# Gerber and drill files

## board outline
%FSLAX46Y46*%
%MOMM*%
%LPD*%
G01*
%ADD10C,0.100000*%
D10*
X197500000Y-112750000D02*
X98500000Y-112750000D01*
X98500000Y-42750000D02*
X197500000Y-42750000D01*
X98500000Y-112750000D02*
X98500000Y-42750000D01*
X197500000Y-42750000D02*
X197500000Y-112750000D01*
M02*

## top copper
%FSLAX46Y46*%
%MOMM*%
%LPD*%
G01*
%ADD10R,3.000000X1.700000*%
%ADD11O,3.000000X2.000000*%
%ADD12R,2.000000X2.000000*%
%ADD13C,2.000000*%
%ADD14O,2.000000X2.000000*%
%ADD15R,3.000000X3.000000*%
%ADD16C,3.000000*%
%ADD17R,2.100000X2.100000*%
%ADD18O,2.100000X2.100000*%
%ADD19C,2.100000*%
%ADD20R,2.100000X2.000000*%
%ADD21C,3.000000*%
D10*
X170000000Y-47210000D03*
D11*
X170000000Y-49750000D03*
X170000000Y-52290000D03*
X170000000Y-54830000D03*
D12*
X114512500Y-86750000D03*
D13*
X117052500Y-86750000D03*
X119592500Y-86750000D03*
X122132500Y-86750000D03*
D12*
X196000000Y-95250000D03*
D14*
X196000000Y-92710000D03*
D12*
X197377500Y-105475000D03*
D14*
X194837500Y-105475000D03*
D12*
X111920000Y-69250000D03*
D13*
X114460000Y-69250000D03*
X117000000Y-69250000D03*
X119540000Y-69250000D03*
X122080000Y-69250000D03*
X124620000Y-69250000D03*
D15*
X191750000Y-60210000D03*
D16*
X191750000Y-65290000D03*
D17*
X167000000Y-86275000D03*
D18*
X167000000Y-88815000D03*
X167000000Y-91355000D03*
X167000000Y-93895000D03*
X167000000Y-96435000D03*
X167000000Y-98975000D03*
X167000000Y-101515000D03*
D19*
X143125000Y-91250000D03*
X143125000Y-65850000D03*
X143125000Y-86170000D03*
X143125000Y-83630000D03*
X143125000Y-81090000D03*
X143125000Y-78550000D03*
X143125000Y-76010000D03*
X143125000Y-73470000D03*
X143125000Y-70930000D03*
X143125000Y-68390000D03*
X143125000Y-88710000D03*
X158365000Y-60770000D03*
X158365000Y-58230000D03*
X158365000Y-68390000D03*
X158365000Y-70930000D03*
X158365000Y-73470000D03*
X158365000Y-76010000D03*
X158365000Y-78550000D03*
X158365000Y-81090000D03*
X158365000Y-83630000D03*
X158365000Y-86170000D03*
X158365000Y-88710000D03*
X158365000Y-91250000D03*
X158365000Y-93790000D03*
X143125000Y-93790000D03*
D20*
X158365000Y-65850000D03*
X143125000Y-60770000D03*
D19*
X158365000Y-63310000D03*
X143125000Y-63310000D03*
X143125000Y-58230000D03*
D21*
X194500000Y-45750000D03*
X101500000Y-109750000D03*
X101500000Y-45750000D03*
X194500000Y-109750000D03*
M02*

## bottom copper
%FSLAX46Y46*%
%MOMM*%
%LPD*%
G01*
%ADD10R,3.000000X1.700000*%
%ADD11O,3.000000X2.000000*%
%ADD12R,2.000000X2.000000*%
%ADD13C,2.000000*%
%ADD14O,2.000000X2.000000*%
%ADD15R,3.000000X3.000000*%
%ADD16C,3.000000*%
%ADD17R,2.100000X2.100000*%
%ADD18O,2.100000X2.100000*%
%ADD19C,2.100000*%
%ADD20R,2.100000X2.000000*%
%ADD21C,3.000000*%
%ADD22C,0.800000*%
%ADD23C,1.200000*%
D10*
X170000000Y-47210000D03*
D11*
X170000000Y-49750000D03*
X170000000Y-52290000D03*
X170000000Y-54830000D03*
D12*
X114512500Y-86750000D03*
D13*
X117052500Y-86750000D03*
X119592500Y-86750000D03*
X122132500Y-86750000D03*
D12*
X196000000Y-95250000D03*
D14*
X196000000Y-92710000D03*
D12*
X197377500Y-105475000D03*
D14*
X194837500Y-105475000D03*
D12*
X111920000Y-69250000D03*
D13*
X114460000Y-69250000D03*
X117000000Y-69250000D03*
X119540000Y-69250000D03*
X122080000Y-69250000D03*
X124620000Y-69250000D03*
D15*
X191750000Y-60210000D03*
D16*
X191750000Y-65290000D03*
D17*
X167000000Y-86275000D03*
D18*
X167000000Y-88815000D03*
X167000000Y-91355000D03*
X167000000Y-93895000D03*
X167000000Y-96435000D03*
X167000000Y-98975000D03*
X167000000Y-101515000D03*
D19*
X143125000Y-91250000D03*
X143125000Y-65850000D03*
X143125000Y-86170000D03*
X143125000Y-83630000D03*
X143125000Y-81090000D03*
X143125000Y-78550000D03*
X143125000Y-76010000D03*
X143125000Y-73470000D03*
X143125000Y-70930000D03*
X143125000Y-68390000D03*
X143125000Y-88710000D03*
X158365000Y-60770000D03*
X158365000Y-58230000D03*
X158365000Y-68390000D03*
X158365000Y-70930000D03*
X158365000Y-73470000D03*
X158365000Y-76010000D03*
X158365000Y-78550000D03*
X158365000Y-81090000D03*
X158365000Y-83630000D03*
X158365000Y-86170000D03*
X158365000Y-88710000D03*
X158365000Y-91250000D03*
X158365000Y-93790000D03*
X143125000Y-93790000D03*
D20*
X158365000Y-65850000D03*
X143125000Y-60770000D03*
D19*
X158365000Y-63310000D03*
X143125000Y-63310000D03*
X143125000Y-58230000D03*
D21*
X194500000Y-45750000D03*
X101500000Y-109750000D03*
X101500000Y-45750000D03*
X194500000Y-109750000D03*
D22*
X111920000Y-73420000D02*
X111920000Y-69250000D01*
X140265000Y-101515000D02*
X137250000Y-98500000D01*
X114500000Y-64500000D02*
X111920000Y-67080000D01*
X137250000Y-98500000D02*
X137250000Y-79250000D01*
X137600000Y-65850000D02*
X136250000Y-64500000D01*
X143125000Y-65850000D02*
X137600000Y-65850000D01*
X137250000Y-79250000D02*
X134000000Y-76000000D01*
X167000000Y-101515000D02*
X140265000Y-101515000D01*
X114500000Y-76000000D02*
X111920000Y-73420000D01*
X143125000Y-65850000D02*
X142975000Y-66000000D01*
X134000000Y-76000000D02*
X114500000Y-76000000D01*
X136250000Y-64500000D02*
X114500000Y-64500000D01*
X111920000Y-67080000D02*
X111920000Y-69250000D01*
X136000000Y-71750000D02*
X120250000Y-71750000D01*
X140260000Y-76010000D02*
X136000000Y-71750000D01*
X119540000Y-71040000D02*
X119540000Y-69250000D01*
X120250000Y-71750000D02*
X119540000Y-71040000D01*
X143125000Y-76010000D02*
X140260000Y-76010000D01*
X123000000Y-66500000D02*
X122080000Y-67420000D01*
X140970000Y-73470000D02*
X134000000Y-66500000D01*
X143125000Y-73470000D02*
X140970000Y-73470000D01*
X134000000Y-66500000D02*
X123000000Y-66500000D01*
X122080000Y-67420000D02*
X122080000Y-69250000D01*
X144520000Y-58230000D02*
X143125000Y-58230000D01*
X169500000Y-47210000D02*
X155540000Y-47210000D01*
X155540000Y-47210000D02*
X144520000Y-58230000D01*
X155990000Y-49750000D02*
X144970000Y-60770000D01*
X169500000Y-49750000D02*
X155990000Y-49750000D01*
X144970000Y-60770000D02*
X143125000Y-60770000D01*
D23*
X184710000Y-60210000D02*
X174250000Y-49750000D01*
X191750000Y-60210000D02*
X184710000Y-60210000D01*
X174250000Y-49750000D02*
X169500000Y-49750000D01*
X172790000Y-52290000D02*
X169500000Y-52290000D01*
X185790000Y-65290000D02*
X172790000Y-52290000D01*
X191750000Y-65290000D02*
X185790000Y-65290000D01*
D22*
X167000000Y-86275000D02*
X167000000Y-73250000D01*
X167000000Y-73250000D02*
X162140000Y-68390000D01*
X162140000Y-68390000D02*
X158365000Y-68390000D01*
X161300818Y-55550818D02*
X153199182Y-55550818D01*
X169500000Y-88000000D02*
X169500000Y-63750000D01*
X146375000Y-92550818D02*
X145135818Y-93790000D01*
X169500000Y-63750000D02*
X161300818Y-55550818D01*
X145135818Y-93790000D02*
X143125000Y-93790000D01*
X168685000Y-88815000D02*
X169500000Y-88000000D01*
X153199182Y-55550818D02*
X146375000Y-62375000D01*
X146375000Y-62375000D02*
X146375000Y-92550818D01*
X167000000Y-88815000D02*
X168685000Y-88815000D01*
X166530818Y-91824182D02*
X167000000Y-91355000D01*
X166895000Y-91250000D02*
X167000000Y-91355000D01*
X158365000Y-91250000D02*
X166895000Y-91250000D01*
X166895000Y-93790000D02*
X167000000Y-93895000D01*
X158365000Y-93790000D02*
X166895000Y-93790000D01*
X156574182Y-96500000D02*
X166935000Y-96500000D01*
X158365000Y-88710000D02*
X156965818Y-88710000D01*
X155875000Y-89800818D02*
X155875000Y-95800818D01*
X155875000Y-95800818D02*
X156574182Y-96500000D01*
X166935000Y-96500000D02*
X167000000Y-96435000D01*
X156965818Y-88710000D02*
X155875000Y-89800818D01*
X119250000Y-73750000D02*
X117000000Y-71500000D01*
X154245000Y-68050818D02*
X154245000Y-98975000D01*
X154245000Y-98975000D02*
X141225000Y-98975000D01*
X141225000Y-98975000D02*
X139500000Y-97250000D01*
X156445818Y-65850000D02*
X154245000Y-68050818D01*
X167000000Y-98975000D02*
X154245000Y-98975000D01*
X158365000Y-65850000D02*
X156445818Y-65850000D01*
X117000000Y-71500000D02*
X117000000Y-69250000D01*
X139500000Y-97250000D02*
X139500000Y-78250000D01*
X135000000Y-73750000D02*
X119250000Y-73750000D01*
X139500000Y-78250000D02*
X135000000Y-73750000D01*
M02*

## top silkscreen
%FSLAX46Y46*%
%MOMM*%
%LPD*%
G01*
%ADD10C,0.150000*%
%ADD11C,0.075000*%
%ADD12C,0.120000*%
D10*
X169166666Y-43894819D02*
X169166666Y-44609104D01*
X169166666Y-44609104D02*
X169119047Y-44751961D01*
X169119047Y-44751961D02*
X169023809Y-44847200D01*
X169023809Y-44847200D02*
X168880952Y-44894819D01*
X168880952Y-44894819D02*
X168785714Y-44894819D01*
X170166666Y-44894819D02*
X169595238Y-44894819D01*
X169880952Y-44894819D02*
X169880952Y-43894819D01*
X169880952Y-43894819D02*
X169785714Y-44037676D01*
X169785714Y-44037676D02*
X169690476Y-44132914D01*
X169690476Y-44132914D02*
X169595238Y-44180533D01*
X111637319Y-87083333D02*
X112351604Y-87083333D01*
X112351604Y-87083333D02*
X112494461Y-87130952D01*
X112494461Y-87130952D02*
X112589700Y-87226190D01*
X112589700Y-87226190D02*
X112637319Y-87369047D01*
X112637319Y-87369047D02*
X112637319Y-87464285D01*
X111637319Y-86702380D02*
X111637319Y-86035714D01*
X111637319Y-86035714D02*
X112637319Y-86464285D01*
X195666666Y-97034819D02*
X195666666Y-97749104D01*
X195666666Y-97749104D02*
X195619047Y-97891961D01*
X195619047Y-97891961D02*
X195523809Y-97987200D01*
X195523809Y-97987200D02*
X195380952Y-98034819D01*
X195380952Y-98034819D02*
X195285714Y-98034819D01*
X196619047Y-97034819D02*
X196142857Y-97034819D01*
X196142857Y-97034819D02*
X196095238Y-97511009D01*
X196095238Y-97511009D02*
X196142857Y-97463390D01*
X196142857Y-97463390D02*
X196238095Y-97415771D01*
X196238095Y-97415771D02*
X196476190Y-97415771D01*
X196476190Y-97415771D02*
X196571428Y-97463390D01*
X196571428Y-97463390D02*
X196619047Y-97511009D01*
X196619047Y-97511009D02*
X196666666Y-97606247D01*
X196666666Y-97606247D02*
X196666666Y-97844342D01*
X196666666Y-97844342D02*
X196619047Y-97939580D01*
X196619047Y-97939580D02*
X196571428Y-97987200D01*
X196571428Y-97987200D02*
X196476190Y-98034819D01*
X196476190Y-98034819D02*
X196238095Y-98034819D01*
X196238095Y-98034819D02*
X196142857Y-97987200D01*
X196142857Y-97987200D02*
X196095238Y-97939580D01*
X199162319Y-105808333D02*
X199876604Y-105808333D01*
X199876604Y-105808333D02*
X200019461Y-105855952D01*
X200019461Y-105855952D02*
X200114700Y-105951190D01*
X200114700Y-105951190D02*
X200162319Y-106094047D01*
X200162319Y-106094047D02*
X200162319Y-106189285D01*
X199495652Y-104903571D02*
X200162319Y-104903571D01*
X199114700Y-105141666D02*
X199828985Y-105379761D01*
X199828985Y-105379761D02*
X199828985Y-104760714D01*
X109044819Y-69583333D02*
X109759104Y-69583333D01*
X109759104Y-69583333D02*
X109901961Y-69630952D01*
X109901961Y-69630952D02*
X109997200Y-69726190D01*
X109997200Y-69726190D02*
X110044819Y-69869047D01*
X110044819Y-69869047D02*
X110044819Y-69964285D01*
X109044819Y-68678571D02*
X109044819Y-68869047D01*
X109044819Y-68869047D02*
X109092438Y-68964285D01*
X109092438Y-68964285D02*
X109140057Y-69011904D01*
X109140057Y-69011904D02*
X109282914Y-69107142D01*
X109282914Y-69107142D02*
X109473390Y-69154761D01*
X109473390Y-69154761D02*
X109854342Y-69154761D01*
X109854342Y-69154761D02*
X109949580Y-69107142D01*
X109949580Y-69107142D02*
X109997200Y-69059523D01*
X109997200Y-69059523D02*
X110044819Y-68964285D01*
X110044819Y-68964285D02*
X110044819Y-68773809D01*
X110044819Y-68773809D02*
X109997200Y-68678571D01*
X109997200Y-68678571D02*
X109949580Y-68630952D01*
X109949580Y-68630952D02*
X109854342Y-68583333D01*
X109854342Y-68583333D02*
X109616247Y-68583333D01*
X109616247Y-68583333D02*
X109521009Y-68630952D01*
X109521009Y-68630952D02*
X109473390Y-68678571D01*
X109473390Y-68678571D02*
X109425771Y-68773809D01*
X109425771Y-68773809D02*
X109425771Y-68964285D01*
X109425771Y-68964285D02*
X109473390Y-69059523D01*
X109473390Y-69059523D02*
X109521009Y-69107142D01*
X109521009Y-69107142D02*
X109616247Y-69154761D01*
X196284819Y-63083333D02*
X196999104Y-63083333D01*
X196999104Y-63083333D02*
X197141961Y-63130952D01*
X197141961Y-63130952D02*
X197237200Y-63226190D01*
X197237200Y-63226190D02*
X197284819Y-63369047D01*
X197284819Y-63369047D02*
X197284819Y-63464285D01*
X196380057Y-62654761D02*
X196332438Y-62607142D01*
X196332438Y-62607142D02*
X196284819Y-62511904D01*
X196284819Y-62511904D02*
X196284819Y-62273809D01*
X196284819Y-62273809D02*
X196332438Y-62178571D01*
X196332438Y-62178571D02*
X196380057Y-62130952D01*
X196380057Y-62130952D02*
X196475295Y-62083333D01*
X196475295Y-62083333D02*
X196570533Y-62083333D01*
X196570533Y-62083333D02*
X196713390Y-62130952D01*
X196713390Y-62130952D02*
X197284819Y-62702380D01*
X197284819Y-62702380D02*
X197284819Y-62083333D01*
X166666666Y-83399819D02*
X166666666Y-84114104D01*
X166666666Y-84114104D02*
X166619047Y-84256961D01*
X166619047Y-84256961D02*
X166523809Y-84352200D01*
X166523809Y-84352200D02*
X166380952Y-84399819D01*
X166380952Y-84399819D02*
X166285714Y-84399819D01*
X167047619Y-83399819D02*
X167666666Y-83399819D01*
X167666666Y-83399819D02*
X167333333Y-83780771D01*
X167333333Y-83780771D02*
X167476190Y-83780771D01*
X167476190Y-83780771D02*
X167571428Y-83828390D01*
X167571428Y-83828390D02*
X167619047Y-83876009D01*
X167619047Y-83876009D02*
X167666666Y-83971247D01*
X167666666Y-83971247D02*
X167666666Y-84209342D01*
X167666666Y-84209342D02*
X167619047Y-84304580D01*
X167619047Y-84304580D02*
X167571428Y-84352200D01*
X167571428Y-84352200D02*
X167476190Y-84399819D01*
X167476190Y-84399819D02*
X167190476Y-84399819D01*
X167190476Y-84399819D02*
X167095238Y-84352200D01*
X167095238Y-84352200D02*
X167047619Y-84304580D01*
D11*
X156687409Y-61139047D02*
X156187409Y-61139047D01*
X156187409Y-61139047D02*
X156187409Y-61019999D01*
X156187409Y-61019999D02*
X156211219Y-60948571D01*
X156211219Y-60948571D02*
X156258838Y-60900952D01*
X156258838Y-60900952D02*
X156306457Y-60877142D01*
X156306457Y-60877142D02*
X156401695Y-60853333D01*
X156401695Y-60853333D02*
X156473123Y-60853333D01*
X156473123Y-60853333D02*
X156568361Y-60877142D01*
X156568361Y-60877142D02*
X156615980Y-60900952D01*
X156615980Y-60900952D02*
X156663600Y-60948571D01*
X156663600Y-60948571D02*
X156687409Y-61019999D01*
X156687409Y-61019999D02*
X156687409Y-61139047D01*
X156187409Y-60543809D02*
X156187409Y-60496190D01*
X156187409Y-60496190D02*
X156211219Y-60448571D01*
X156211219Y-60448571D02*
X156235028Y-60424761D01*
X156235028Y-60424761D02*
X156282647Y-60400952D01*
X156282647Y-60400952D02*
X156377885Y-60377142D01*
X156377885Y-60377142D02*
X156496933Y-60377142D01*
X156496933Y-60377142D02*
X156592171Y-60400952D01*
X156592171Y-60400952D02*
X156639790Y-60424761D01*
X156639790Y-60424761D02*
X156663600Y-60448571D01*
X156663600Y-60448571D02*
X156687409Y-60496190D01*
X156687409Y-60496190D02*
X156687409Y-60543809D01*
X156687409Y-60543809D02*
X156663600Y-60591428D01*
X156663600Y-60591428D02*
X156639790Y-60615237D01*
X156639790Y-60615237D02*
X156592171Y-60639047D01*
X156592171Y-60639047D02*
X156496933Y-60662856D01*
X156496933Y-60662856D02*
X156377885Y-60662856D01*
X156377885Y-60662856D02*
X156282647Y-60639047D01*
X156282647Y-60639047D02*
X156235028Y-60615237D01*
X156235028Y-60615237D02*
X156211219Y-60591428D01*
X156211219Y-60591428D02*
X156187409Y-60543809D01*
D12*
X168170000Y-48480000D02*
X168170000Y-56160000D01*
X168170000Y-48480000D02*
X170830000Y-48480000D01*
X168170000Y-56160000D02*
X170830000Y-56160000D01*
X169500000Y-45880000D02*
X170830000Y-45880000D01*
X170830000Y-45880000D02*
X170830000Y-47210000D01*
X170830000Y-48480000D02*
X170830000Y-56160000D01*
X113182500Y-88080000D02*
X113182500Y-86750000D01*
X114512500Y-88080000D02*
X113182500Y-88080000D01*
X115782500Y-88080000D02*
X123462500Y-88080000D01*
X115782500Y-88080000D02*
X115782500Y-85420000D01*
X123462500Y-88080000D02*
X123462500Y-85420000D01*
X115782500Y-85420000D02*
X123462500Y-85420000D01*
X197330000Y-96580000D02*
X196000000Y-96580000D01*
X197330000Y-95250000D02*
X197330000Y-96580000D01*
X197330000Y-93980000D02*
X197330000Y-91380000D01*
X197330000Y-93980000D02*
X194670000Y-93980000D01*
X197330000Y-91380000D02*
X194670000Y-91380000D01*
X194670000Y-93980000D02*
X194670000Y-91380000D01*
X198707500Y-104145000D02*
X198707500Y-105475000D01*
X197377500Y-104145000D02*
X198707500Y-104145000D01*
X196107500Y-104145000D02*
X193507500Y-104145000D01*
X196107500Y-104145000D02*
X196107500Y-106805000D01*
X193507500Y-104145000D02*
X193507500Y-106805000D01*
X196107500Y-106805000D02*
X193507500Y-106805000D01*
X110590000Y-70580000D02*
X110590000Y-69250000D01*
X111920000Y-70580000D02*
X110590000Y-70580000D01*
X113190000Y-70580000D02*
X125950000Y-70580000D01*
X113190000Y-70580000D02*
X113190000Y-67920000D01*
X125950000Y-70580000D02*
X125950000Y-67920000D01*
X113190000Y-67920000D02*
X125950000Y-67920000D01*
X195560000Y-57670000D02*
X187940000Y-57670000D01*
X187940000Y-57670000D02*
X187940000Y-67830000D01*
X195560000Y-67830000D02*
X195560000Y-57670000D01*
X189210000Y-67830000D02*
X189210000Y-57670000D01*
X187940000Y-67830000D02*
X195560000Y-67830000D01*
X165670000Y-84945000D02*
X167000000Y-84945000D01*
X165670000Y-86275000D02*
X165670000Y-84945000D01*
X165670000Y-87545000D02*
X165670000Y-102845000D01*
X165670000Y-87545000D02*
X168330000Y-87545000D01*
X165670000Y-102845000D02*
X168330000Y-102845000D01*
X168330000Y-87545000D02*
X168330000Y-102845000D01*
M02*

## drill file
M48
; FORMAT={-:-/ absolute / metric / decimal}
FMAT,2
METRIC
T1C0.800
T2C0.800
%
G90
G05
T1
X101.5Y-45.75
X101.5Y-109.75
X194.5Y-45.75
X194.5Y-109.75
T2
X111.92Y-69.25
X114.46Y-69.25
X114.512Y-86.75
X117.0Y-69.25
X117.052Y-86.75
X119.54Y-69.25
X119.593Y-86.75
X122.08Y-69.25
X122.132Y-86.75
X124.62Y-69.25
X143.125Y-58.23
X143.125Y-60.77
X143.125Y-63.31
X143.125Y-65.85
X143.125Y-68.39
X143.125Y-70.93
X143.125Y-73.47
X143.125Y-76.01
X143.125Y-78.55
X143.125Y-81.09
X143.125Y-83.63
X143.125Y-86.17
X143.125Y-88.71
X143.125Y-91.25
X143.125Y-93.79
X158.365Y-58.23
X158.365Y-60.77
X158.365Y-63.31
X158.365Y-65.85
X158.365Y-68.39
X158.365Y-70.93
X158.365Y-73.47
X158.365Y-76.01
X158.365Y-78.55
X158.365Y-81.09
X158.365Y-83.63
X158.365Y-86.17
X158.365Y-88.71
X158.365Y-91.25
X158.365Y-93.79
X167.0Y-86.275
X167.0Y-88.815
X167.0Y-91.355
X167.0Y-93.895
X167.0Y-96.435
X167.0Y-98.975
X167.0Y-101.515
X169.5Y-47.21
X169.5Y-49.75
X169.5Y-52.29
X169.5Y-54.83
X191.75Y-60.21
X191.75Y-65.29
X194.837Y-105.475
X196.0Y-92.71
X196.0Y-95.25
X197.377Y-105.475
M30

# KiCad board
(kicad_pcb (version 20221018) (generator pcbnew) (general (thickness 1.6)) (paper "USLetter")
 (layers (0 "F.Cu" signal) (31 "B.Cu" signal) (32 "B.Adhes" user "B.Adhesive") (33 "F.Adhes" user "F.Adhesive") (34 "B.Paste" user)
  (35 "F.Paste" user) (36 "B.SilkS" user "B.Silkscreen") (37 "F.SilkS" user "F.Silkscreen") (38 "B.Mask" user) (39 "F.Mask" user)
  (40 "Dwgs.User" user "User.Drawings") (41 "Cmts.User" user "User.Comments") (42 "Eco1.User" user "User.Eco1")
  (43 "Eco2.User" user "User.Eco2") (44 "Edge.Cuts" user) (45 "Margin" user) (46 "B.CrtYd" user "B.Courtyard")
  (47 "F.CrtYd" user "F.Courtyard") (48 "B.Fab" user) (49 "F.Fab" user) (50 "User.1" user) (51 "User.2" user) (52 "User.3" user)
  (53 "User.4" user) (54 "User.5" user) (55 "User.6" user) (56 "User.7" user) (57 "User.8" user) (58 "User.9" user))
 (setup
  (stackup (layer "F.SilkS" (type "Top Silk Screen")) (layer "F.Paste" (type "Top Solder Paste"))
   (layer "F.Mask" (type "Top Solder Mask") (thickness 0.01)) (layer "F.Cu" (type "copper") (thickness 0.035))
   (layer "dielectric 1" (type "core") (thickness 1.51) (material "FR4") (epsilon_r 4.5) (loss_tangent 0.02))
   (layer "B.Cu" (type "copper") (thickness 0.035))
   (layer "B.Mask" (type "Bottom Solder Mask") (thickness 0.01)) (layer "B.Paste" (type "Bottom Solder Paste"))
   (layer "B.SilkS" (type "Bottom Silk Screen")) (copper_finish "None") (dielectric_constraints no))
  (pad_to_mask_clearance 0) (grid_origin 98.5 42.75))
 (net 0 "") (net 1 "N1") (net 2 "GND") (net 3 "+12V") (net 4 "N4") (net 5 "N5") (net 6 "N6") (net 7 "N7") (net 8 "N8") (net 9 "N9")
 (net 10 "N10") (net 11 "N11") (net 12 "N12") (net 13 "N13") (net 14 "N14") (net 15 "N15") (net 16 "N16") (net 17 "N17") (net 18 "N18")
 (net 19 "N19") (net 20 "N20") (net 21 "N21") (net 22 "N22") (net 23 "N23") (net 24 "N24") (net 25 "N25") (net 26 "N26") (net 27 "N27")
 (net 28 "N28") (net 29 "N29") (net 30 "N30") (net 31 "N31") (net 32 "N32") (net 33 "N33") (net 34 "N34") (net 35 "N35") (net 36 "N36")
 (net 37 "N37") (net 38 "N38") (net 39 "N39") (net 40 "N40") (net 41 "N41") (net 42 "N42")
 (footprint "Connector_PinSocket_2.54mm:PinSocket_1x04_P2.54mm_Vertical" (layer "F.Cu") (at 169.5 47.21)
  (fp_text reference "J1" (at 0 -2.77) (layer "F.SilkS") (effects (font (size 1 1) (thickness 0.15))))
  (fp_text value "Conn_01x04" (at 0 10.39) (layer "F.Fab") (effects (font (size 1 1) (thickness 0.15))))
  (fp_line (start -1.33 1.27) (end -1.33 8.95) (stroke (width 0.12) (type solid)) (layer "F.SilkS"))
  (fp_line (start -1.33 1.27) (end 1.33 1.27) (stroke (width 0.12) (type solid)) (layer "F.SilkS"))
  (fp_line (start -1.33 8.95) (end 1.33 8.95) (stroke (width 0.12) (type solid)) (layer "F.SilkS"))
  (fp_line (start 0 -1.33) (end 1.33 -1.33) (stroke (width 0.12) (type solid)) (layer "F.SilkS"))
  (fp_line (start 1.33 -1.33) (end 1.33 0) (stroke (width 0.12) (type solid)) (layer "F.SilkS"))
  (fp_line (start 1.33 1.27) (end 1.33 8.95) (stroke (width 0.12) (type solid)) (layer "F.SilkS"))
  (pad "1" thru_hole rect (at 0 0) (size 3 1.7) (drill 0.8 (offset 0.5 0)) (layers "*.Cu" "*.Mask") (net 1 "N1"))
  (pad "2" thru_hole oval (at 0 2.54) (size 3 2) (drill 0.8 (offset 0.5 0)) (layers "*.Cu" "*.Mask") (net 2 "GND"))
  (pad "3" thru_hole oval (at 0 5.08) (size 3 2) (drill 0.8 (offset 0.5 0)) (layers "*.Cu" "*.Mask") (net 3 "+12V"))
  (pad "4" thru_hole oval (at 0 7.62) (size 3 2) (drill 0.8 (offset 0.5 0)) (layers "*.Cu" "*.Mask") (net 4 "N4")))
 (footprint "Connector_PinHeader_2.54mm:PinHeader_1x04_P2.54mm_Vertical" (layer "F.Cu") (at 114.5125 86.75 90)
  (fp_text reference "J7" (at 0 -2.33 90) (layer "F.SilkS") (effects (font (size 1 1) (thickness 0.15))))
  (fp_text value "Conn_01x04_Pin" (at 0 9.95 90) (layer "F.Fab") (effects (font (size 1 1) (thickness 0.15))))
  (fp_line (start -1.33 -1.33) (end 0 -1.33) (stroke (width 0.12) (type solid)) (layer "F.SilkS"))
  (fp_line (start -1.33 0) (end -1.33 -1.33) (stroke (width 0.12) (type solid)) (layer "F.SilkS"))
  (fp_line (start -1.33 1.27) (end -1.33 8.95) (stroke (width 0.12) (type solid)) (layer "F.SilkS"))
  (fp_line (start -1.33 1.27) (end 1.33 1.27) (stroke (width 0.12) (type solid)) (layer "F.SilkS"))
  (fp_line (start -1.33 8.95) (end 1.33 8.95) (stroke (width 0.12) (type solid)) (layer "F.SilkS"))
  (fp_line (start 1.33 1.27) (end 1.33 8.95) (stroke (width 0.12) (type solid)) (layer "F.SilkS"))
  (pad "1" thru_hole rect (at 0 0 90) (size 2 2) (drill 0.8) (layers "*.Cu" "*.Mask") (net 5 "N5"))
  (pad "2" thru_hole circle (at 0 2.54 90) (size 2 2) (drill 0.8) (layers "*.Cu" "*.Mask") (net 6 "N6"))
  (pad "3" thru_hole circle (at 0 5.08 90) (size 2 2) (drill 0.8) (layers "*.Cu" "*.Mask") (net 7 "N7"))
  (pad "4" thru_hole circle (at 0 7.62 90) (size 2 2) (drill 0.8) (layers "*.Cu" "*.Mask") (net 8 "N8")))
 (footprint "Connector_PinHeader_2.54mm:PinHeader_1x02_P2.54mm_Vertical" (layer "F.Cu") (at 196 95.25 180)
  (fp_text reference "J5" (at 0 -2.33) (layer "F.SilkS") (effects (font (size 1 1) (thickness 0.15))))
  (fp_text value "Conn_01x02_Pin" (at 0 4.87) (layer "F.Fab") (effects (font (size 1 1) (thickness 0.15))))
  (fp_line (start -1.33 -1.33) (end 0 -1.33) (stroke (width 0.12) (type solid)) (layer "F.SilkS"))
  (fp_line (start -1.33 0) (end -1.33 -1.33) (stroke (width 0.12) (type solid)) (layer "F.SilkS"))
  (fp_line (start -1.33 1.27) (end -1.33 3.87) (stroke (width 0.12) (type solid)) (layer "F.SilkS"))
  (fp_line (start -1.33 1.27) (end 1.33 1.27) (stroke (width 0.12) (type solid)) (layer "F.SilkS"))
  (fp_line (start -1.33 3.87) (end 1.33 3.87) (stroke (width 0.12) (type solid)) (layer "F.SilkS"))
  (fp_line (start 1.33 1.27) (end 1.33 3.87) (stroke (width 0.12) (type solid)) (layer "F.SilkS"))
  (pad "1" thru_hole rect (at 0 0 180) (size 2 2) (drill 0.8) (layers "*.Cu" "*.Mask") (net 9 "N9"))
  (pad "2" thru_hole oval (at 0 2.54 180) (size 2 2) (drill 0.8) (layers "*.Cu" "*.Mask") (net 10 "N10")))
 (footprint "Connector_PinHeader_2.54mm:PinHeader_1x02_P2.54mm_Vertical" (layer "F.Cu") (at 197.3775 105.475 -90)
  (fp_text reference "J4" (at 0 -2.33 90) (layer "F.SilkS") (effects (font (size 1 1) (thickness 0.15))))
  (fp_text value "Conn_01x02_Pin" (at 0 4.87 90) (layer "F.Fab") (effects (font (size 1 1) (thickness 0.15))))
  (fp_line (start -1.33 -1.33) (end 0 -1.33) (stroke (width 0.12) (type solid)) (layer "F.SilkS"))
  (fp_line (start -1.33 0) (end -1.33 -1.33) (stroke (width 0.12) (type solid)) (layer "F.SilkS"))
  (fp_line (start -1.33 1.27) (end -1.33 3.87) (stroke (width 0.12) (type solid)) (layer "F.SilkS"))
  (fp_line (start -1.33 1.27) (end 1.33 1.27) (stroke (width 0.12) (type solid)) (layer "F.SilkS"))
  (fp_line (start -1.33 3.87) (end 1.33 3.87) (stroke (width 0.12) (type solid)) (layer "F.SilkS"))
  (fp_line (start 1.33 1.27) (end 1.33 3.87) (stroke (width 0.12) (type solid)) (layer "F.SilkS"))
  (pad "1" thru_hole rect (at 0 0 270) (size 2 2) (drill 0.8) (layers "*.Cu" "*.Mask") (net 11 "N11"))
  (pad "2" thru_hole oval (at 0 2.54 270) (size 2 2) (drill 0.8) (layers "*.Cu" "*.Mask") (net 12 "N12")))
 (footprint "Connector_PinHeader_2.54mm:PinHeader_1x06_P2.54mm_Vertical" (layer "F.Cu") (at 111.92 69.25 90)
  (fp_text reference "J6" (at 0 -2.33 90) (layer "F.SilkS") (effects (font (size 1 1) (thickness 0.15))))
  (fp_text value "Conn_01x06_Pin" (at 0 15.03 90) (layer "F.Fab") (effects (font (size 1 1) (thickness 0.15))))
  (fp_line (start -1.33 -1.33) (end 0 -1.33) (stroke (width 0.12) (type solid)) (layer "F.SilkS"))
  (fp_line (start -1.33 0) (end -1.33 -1.33) (stroke (width 0.12) (type solid)) (layer "F.SilkS"))
  (fp_line (start -1.33 1.27) (end -1.33 14.03) (stroke (width 0.12) (type solid)) (layer "F.SilkS"))
  (fp_line (start -1.33 1.27) (end 1.33 1.27) (stroke (width 0.12) (type solid)) (layer "F.SilkS"))
  (fp_line (start -1.33 14.03) (end 1.33 14.03) (stroke (width 0.12) (type solid)) (layer "F.SilkS"))
  (fp_line (start 1.33 1.27) (end 1.33 14.03) (stroke (width 0.12) (type solid)) (layer "F.SilkS"))
  (pad "1" thru_hole rect (at 0 0 90) (size 2 2) (drill 0.8) (layers "*.Cu" "*.Mask") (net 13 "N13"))
  (pad "2" thru_hole circle (at 0 2.54 90) (size 2 2) (drill 0.8) (layers "*.Cu" "*.Mask") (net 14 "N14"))
  (pad "3" thru_hole circle (at 0 5.08 90) (size 2 2) (drill 0.8) (layers "*.Cu" "*.Mask") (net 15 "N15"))
  (pad "4" thru_hole circle (at 0 7.62 90) (size 2 2) (drill 0.8) (layers "*.Cu" "*.Mask") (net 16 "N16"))
  (pad "5" thru_hole circle (at 0 10.16 90) (size 2 2) (drill 0.8) (layers "*.Cu" "*.Mask") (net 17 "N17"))
  (pad "6" thru_hole circle (at 0 12.7 90) (size 2 2) (drill 0.8) (layers "*.Cu" "*.Mask") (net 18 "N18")))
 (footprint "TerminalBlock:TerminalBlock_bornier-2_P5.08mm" (layer "F.Cu") (at 191.75 60.21 -90)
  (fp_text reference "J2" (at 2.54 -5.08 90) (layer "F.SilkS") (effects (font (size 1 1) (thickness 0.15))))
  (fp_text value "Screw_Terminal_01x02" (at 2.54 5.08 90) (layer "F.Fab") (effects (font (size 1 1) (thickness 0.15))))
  (fp_line (start -2.54 -3.81) (end -2.54 3.81) (stroke (width 0.12) (type solid)) (layer "F.SilkS"))
  (fp_line (start -2.54 3.81) (end 7.62 3.81) (stroke (width 0.12) (type solid)) (layer "F.SilkS"))
  (fp_line (start 7.62 -3.81) (end -2.54 -3.81) (stroke (width 0.12) (type solid)) (layer "F.SilkS"))
  (fp_line (start 7.62 2.54) (end -2.54 2.54) (stroke (width 0.12) (type solid)) (layer "F.SilkS"))
  (fp_line (start 7.62 3.81) (end 7.62 -3.81) (stroke (width 0.12) (type solid)) (layer "F.SilkS"))
  (pad "1" thru_hole rect (at 0 0 270) (size 3 3) (drill 0.8) (layers "*.Cu" "*.Mask") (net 2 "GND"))
  (pad "2" thru_hole circle (at 5.08 0 270) (size 3 3) (drill 0.8) (layers "*.Cu" "*.Mask") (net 3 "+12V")))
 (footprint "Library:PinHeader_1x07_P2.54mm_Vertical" (layer "F.Cu") (at 167 86.275)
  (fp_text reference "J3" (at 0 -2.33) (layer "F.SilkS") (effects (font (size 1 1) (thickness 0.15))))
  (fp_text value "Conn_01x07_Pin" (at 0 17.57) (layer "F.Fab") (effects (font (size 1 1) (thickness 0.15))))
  (fp_line (start -1.33 -1.33) (end 0 -1.33) (stroke (width 0.12) (type solid)) (layer "F.SilkS"))
  (fp_line (start -1.33 0) (end -1.33 -1.33) (stroke (width 0.12) (type solid)) (layer "F.SilkS"))
  (fp_line (start -1.33 1.27) (end -1.33 16.57) (stroke (width 0.12) (type solid)) (layer "F.SilkS"))
  (fp_line (start -1.33 1.27) (end 1.33 1.27) (stroke (width 0.12) (type solid)) (layer "F.SilkS"))
  (fp_line (start -1.33 16.57) (end 1.33 16.57) (stroke (width 0.12) (type solid)) (layer "F.SilkS"))
  (fp_line (start 1.33 1.27) (end 1.33 16.57) (stroke (width 0.12) (type solid)) (layer "F.SilkS"))
  (pad "1" thru_hole rect (at 0 0) (size 2.1 2.1) (drill 0.8) (layers "*.Cu" "*.Mask") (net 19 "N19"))
  (pad "2" thru_hole oval (at 0 2.54) (size 2.1 2.1) (drill 0.8) (layers "*.Cu" "*.Mask") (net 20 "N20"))
  (pad "3" thru_hole oval (at 0 5.08) (size 2.1 2.1) (drill 0.8) (layers "*.Cu" "*.Mask") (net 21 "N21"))
  (pad "4" thru_hole oval (at 0 7.62) (size 2.1 2.1) (drill 0.8) (layers "*.Cu" "*.Mask") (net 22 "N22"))
  (pad "5" thru_hole oval (at 0 10.16) (size 2.1 2.1) (drill 0.8) (layers "*.Cu" "*.Mask") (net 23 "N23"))
  (pad "6" thru_hole oval (at 0 12.7) (size 2.1 2.1) (drill 0.8) (layers "*.Cu" "*.Mask") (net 15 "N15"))
  (pad "7" thru_hole oval (at 0 15.24) (size 2.1 2.1) (drill 0.8) (layers "*.Cu" "*.Mask") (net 13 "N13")))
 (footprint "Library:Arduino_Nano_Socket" (layer "B.Cu") (at 150.745 97.6 180)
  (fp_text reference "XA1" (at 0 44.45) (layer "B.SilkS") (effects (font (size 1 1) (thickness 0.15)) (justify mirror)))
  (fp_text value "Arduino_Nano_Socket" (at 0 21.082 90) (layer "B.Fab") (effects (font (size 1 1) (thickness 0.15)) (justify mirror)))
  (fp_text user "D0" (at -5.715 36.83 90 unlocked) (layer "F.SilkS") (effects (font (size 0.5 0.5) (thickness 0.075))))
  (pad "3V3" thru_hole circle (at 7.62 6.35 180) (size 2.1 2.1) (drill 0.8) (layers "*.Cu" "*.Mask") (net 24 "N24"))
  (pad "5V" thru_hole circle (at 7.62 31.75 180) (size 2.1 2.1) (drill 0.8) (layers "*.Cu" "*.Mask") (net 13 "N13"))
  (pad "A0" thru_hole circle (at 7.62 11.43 180) (size 2.1 2.1) (drill 0.8) (layers "*.Cu" "*.Mask") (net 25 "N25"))
  (pad "A1" thru_hole circle (at 7.62 13.97 180) (size 2.1 2.1) (drill 0.8) (layers "*.Cu" "*.Mask") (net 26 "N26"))
  (pad "A2" thru_hole circle (at 7.62 16.51 180) (size 2.1 2.1) (drill 0.8) (layers "*.Cu" "*.Mask") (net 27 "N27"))
  (pad "A3" thru_hole circle (at 7.62 19.05 180) (size 2.1 2.1) (drill 0.8) (layers "*.Cu" "*.Mask") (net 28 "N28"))
  (pad "A4" thru_hole circle (at 7.62 21.59 180) (size 2.1 2.1) (drill 0.8) (layers "*.Cu" "*.Mask") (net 16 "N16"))
  (pad "A5" thru_hole circle (at 7.62 24.13 180) (size 2.1 2.1) (drill 0.8) (layers "*.Cu" "*.Mask") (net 17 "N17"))
  (pad "A6" thru_hole circle (at 7.62 26.67 180) (size 2.1 2.1) (drill 0.8) (layers "*.Cu" "*.Mask") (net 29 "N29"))
  (pad "A7" thru_hole circle (at 7.62 29.21 180) (size 2.1 2.1) (drill 0.8) (layers "*.Cu" "*.Mask") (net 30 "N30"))
  (pad "AREF" thru_hole circle (at 7.62 8.89 180) (size 2.1 2.1) (drill 0.8) (layers "*.Cu" "*.Mask") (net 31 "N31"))
  (pad "D0" thru_hole circle (at -7.62 36.83 180) (size 2.1 2.1) (drill 0.8) (layers "*.Cu" "*.Mask") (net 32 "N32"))
  (pad "D1" thru_hole circle (at -7.62 39.37 180) (size 2.1 2.1) (drill 0.8) (layers "*.Cu" "*.Mask") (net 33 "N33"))
  (pad "D2" thru_hole circle (at -7.62 29.21 180) (size 2.1 2.1) (drill 0.8) (layers "*.Cu" "*.Mask") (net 19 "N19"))
  (pad "D3" thru_hole circle (at -7.62 26.67 180) (size 2.1 2.1) (drill 0.8) (layers "*.Cu" "*.Mask") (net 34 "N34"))
  (pad "D4" thru_hole circle (at -7.62 24.13 180) (size 2.1 2.1) (drill 0.8) (layers "*.Cu" "*.Mask") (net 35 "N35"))
  (pad "D5" thru_hole circle (at -7.62 21.59 180) (size 2.1 2.1) (drill 0.8) (layers "*.Cu" "*.Mask") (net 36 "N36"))
  (pad "D6" thru_hole circle (at -7.62 19.05 180) (size 2.1 2.1) (drill 0.8) (layers "*.Cu" "*.Mask") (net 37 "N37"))
  (pad "D7" thru_hole circle (at -7.62 16.51 180) (size 2.1 2.1) (drill 0.8) (layers "*.Cu" "*.Mask") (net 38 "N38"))
  (pad "D8" thru_hole circle (at -7.62 13.97 180) (size 2.1 2.1) (drill 0.8) (layers "*.Cu" "*.Mask") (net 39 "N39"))
  (pad "D9" thru_hole circle (at -7.62 11.43 180) (size 2.1 2.1) (drill 0.8) (layers "*.Cu" "*.Mask") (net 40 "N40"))
  (pad "D10" thru_hole circle (at -7.62 8.89 180) (size 2.1 2.1) (drill 0.8) (layers "*.Cu" "*.Mask") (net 23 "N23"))
  (pad "D11" thru_hole circle (at -7.62 6.35 180) (size 2.1 2.1) (drill 0.8) (layers "*.Cu" "*.Mask") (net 21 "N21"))
  (pad "D12" thru_hole circle (at -7.62 3.81 180) (size 2.1 2.1) (drill 0.8) (layers "*.Cu" "*.Mask") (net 22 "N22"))
  (pad "D13" thru_hole circle (at 7.62 3.81 180) (size 2.1 2.1) (drill 0.8) (layers "*.Cu" "*.Mask") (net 20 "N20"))
  (pad "GND1" thru_hole rect (at -7.62 31.75 180) (size 2.1 2) (drill 0.8) (layers "*.Cu" "*.Mask") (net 15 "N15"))
  (pad "GND2" thru_hole rect (at 7.62 36.83 180) (size 2.1 2) (drill 0.8) (layers "*.Cu" "*.Mask") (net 2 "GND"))
  (pad "RST1" thru_hole circle (at -7.62 34.29 180) (size 2.1 2.1) (drill 0.8) (layers "*.Cu" "*.Mask") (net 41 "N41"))
  (pad "RST2" thru_hole circle (at 7.62 34.29 180) (size 2.1 2.1) (drill 0.8) (layers "*.Cu" "*.Mask") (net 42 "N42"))
  (pad "VIN" thru_hole circle (at 7.62 39.37 180) (size 2.1 2.1) (drill 0.8) (layers "*.Cu" "*.Mask") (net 1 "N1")))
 (gr_line (start 197.5 112.75) (end 98.5 112.75) (stroke (width 0.1) (type default)) (layer "Edge.Cuts"))
 (gr_line (start 98.5 42.75) (end 197.5 42.75) (stroke (width 0.1) (type default)) (layer "Edge.Cuts"))
 (gr_line (start 98.5 112.75) (end 98.5 42.75) (stroke (width 0.1) (type default)) (layer "Edge.Cuts"))
 (gr_line (start 197.5 42.75) (end 197.5 112.75) (stroke (width 0.1) (type default)) (layer "Edge.Cuts"))
 (via (at 194.5 45.75) (size 3) (drill 0.8) (layers "F.Cu" "B.Cu") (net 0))
 (via (at 101.5 109.75) (size 3) (drill 0.8) (layers "F.Cu" "B.Cu") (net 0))
 (via (at 101.5 45.75) (size 3) (drill 0.8) (layers "F.Cu" "B.Cu") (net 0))
 (via (at 194.5 109.75) (size 3) (drill 0.8) (layers "F.Cu" "B.Cu") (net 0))
 (segment (start 111.92 73.42) (end 111.92 69.25) (width 0.8) (layer "B.Cu") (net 13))
 (segment (start 140.265 101.515) (end 137.25 98.5) (width 0.8) (layer "B.Cu") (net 13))
 (segment (start 114.5 64.5) (end 111.92 67.08) (width 0.8) (layer "B.Cu") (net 13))
 (segment (start 137.25 98.5) (end 137.25 79.25) (width 0.8) (layer "B.Cu") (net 13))
 (segment (start 137.6 65.85) (end 136.25 64.5) (width 0.8) (layer "B.Cu") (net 13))
 (segment (start 143.125 65.85) (end 137.6 65.85) (width 0.8) (layer "B.Cu") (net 13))
 (segment (start 137.25 79.25) (end 134 76) (width 0.8) (layer "B.Cu") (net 13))
 (segment (start 167 101.515) (end 140.265 101.515) (width 0.8) (layer "B.Cu") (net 13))
 (segment (start 114.5 76) (end 111.92 73.42) (width 0.8) (layer "B.Cu") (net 13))
 (segment (start 143.125 65.85) (end 142.975 66) (width 0.8) (layer "B.Cu") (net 13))
 (segment (start 134 76) (end 114.5 76) (width 0.8) (layer "B.Cu") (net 13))
 (segment (start 136.25 64.5) (end 114.5 64.5) (width 0.8) (layer "B.Cu") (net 13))
 (segment (start 111.92 67.08) (end 111.92 69.25) (width 0.8) (layer "B.Cu") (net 13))
 (segment (start 136 71.75) (end 120.25 71.75) (width 0.8) (layer "B.Cu") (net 16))
 (segment (start 140.26 76.01) (end 136 71.75) (width 0.8) (layer "B.Cu") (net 16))
 (segment (start 119.54 71.04) (end 119.54 69.25) (width 0.8) (layer "B.Cu") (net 16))
 (segment (start 120.25 71.75) (end 119.54 71.04) (width 0.8) (layer "B.Cu") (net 16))
 (segment (start 143.125 76.01) (end 140.26 76.01) (width 0.8) (layer "B.Cu") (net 16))
 (segment (start 123 66.5) (end 122.08 67.42) (width 0.8) (layer "B.Cu") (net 17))
 (segment (start 140.97 73.47) (end 134 66.5) (width 0.8) (layer "B.Cu") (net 17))
 (segment (start 143.125 73.47) (end 140.97 73.47) (width 0.8) (layer "B.Cu") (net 17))
 (segment (start 134 66.5) (end 123 66.5) (width 0.8) (layer "B.Cu") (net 17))
 (segment (start 122.08 67.42) (end 122.08 69.25) (width 0.8) (layer "B.Cu") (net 17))
 (segment (start 144.52 58.23) (end 143.125 58.23) (width 0.8) (layer "B.Cu") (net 1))
 (segment (start 169.5 47.21) (end 155.54 47.21) (width 0.8) (layer "B.Cu") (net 1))
 (segment (start 155.54 47.21) (end 144.52 58.23) (width 0.8) (layer "B.Cu") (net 1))
 (segment (start 155.99 49.75) (end 144.97 60.77) (width 0.8) (layer "B.Cu") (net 2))
 (segment (start 169.5 49.75) (end 155.99 49.75) (width 0.8) (layer "B.Cu") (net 2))
 (segment (start 144.97 60.77) (end 143.125 60.77) (width 0.8) (layer "B.Cu") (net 2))
 (segment (start 184.71 60.21) (end 174.25 49.75) (width 1.2) (layer "B.Cu") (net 2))
 (segment (start 191.75 60.21) (end 184.71 60.21) (width 1.2) (layer "B.Cu") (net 2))
 (segment (start 174.25 49.75) (end 169.5 49.75) (width 1.2) (layer "B.Cu") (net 2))
 (segment (start 172.79 52.29) (end 169.5 52.29) (width 1.2) (layer "B.Cu") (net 3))
 (segment (start 185.79 65.29) (end 172.79 52.29) (width 1.2) (layer "B.Cu") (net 3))
 (segment (start 191.75 65.29) (end 185.79 65.29) (width 1.2) (layer "B.Cu") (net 3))
 (segment (start 167 86.275) (end 167 73.25) (width 0.8) (layer "B.Cu") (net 19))
 (segment (start 167 73.25) (end 162.14 68.39) (width 0.8) (layer "B.Cu") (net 19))
 (segment (start 162.14 68.39) (end 158.365 68.39) (width 0.8) (layer "B.Cu") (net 19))
 (segment (start 161.300818 55.550818) (end 153.199182 55.550818) (width 0.8) (layer "B.Cu") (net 20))
 (segment (start 169.5 88) (end 169.5 63.75) (width 0.8) (layer "B.Cu") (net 20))
 (segment (start 146.375 92.550818) (end 145.135818 93.79) (width 0.8) (layer "B.Cu") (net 20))
 (segment (start 169.5 63.75) (end 161.300818 55.550818) (width 0.8) (layer "B.Cu") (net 20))
 (segment (start 145.135818 93.79) (end 143.125 93.79) (width 0.8) (layer "B.Cu") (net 20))
 (segment (start 168.685 88.815) (end 169.5 88) (width 0.8) (layer "B.Cu") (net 20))
 (segment (start 153.199182 55.550818) (end 146.375 62.375) (width 0.8) (layer "B.Cu") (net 20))
 (segment (start 146.375 62.375) (end 146.375 92.550818) (width 0.8) (layer "B.Cu") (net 20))
 (segment (start 167 88.815) (end 168.685 88.815) (width 0.8) (layer "B.Cu") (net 20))
 (segment (start 166.530818 91.824182) (end 167 91.355) (width 0.8) (layer "B.Cu") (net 21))
 (segment (start 166.895 91.25) (end 167 91.355) (width 0.8) (layer "B.Cu") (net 21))
 (segment (start 158.365 91.25) (end 166.895 91.25) (width 0.8) (layer "B.Cu") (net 21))
 (segment (start 166.895 93.79) (end 167 93.895) (width 0.8) (layer "B.Cu") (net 22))
 (segment (start 158.365 93.79) (end 166.895 93.79) (width 0.8) (layer "B.Cu") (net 22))
 (segment (start 156.574182 96.5) (end 166.935 96.5) (width 0.8) (layer "B.Cu") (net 23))
 (segment (start 158.365 88.71) (end 156.965818 88.71) (width 0.8) (layer "B.Cu") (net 23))
 (segment (start 155.875 89.800818) (end 155.875 95.800818) (width 0.8) (layer "B.Cu") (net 23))
 (segment (start 155.875 95.800818) (end 156.574182 96.5) (width 0.8) (layer "B.Cu") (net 23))
 (segment (start 166.935 96.5) (end 167 96.435) (width 0.8) (layer "B.Cu") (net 23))
 (segment (start 156.965818 88.71) (end 155.875 89.800818) (width 0.8) (layer "B.Cu") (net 23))
 (segment (start 119.25 73.75) (end 117 71.5) (width 0.8) (layer "B.Cu") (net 15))
 (segment (start 154.245 68.050818) (end 154.245 98.975) (width 0.8) (layer "B.Cu") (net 15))
 (segment (start 154.245 98.975) (end 141.225 98.975) (width 0.8) (layer "B.Cu") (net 15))
 (segment (start 141.225 98.975) (end 139.5 97.25) (width 0.8) (layer "B.Cu") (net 15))
 (segment (start 156.445818 65.85) (end 154.245 68.050818) (width 0.8) (layer "B.Cu") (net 15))
 (segment (start 167 98.975) (end 154.245 98.975) (width 0.8) (layer "B.Cu") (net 15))
 (segment (start 158.365 65.85) (end 156.445818 65.85) (width 0.8) (layer "B.Cu") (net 15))
 (segment (start 117 71.5) (end 117 69.25) (width 0.8) (layer "B.Cu") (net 15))
 (segment (start 139.5 97.25) (end 139.5 78.25) (width 0.8) (layer "B.Cu") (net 15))
 (segment (start 135 73.75) (end 119.25 73.75) (width 0.8) (layer "B.Cu") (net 15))
 (segment (start 139.5 78.25) (end 135 73.75) (width 0.8) (layer "B.Cu") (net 15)))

